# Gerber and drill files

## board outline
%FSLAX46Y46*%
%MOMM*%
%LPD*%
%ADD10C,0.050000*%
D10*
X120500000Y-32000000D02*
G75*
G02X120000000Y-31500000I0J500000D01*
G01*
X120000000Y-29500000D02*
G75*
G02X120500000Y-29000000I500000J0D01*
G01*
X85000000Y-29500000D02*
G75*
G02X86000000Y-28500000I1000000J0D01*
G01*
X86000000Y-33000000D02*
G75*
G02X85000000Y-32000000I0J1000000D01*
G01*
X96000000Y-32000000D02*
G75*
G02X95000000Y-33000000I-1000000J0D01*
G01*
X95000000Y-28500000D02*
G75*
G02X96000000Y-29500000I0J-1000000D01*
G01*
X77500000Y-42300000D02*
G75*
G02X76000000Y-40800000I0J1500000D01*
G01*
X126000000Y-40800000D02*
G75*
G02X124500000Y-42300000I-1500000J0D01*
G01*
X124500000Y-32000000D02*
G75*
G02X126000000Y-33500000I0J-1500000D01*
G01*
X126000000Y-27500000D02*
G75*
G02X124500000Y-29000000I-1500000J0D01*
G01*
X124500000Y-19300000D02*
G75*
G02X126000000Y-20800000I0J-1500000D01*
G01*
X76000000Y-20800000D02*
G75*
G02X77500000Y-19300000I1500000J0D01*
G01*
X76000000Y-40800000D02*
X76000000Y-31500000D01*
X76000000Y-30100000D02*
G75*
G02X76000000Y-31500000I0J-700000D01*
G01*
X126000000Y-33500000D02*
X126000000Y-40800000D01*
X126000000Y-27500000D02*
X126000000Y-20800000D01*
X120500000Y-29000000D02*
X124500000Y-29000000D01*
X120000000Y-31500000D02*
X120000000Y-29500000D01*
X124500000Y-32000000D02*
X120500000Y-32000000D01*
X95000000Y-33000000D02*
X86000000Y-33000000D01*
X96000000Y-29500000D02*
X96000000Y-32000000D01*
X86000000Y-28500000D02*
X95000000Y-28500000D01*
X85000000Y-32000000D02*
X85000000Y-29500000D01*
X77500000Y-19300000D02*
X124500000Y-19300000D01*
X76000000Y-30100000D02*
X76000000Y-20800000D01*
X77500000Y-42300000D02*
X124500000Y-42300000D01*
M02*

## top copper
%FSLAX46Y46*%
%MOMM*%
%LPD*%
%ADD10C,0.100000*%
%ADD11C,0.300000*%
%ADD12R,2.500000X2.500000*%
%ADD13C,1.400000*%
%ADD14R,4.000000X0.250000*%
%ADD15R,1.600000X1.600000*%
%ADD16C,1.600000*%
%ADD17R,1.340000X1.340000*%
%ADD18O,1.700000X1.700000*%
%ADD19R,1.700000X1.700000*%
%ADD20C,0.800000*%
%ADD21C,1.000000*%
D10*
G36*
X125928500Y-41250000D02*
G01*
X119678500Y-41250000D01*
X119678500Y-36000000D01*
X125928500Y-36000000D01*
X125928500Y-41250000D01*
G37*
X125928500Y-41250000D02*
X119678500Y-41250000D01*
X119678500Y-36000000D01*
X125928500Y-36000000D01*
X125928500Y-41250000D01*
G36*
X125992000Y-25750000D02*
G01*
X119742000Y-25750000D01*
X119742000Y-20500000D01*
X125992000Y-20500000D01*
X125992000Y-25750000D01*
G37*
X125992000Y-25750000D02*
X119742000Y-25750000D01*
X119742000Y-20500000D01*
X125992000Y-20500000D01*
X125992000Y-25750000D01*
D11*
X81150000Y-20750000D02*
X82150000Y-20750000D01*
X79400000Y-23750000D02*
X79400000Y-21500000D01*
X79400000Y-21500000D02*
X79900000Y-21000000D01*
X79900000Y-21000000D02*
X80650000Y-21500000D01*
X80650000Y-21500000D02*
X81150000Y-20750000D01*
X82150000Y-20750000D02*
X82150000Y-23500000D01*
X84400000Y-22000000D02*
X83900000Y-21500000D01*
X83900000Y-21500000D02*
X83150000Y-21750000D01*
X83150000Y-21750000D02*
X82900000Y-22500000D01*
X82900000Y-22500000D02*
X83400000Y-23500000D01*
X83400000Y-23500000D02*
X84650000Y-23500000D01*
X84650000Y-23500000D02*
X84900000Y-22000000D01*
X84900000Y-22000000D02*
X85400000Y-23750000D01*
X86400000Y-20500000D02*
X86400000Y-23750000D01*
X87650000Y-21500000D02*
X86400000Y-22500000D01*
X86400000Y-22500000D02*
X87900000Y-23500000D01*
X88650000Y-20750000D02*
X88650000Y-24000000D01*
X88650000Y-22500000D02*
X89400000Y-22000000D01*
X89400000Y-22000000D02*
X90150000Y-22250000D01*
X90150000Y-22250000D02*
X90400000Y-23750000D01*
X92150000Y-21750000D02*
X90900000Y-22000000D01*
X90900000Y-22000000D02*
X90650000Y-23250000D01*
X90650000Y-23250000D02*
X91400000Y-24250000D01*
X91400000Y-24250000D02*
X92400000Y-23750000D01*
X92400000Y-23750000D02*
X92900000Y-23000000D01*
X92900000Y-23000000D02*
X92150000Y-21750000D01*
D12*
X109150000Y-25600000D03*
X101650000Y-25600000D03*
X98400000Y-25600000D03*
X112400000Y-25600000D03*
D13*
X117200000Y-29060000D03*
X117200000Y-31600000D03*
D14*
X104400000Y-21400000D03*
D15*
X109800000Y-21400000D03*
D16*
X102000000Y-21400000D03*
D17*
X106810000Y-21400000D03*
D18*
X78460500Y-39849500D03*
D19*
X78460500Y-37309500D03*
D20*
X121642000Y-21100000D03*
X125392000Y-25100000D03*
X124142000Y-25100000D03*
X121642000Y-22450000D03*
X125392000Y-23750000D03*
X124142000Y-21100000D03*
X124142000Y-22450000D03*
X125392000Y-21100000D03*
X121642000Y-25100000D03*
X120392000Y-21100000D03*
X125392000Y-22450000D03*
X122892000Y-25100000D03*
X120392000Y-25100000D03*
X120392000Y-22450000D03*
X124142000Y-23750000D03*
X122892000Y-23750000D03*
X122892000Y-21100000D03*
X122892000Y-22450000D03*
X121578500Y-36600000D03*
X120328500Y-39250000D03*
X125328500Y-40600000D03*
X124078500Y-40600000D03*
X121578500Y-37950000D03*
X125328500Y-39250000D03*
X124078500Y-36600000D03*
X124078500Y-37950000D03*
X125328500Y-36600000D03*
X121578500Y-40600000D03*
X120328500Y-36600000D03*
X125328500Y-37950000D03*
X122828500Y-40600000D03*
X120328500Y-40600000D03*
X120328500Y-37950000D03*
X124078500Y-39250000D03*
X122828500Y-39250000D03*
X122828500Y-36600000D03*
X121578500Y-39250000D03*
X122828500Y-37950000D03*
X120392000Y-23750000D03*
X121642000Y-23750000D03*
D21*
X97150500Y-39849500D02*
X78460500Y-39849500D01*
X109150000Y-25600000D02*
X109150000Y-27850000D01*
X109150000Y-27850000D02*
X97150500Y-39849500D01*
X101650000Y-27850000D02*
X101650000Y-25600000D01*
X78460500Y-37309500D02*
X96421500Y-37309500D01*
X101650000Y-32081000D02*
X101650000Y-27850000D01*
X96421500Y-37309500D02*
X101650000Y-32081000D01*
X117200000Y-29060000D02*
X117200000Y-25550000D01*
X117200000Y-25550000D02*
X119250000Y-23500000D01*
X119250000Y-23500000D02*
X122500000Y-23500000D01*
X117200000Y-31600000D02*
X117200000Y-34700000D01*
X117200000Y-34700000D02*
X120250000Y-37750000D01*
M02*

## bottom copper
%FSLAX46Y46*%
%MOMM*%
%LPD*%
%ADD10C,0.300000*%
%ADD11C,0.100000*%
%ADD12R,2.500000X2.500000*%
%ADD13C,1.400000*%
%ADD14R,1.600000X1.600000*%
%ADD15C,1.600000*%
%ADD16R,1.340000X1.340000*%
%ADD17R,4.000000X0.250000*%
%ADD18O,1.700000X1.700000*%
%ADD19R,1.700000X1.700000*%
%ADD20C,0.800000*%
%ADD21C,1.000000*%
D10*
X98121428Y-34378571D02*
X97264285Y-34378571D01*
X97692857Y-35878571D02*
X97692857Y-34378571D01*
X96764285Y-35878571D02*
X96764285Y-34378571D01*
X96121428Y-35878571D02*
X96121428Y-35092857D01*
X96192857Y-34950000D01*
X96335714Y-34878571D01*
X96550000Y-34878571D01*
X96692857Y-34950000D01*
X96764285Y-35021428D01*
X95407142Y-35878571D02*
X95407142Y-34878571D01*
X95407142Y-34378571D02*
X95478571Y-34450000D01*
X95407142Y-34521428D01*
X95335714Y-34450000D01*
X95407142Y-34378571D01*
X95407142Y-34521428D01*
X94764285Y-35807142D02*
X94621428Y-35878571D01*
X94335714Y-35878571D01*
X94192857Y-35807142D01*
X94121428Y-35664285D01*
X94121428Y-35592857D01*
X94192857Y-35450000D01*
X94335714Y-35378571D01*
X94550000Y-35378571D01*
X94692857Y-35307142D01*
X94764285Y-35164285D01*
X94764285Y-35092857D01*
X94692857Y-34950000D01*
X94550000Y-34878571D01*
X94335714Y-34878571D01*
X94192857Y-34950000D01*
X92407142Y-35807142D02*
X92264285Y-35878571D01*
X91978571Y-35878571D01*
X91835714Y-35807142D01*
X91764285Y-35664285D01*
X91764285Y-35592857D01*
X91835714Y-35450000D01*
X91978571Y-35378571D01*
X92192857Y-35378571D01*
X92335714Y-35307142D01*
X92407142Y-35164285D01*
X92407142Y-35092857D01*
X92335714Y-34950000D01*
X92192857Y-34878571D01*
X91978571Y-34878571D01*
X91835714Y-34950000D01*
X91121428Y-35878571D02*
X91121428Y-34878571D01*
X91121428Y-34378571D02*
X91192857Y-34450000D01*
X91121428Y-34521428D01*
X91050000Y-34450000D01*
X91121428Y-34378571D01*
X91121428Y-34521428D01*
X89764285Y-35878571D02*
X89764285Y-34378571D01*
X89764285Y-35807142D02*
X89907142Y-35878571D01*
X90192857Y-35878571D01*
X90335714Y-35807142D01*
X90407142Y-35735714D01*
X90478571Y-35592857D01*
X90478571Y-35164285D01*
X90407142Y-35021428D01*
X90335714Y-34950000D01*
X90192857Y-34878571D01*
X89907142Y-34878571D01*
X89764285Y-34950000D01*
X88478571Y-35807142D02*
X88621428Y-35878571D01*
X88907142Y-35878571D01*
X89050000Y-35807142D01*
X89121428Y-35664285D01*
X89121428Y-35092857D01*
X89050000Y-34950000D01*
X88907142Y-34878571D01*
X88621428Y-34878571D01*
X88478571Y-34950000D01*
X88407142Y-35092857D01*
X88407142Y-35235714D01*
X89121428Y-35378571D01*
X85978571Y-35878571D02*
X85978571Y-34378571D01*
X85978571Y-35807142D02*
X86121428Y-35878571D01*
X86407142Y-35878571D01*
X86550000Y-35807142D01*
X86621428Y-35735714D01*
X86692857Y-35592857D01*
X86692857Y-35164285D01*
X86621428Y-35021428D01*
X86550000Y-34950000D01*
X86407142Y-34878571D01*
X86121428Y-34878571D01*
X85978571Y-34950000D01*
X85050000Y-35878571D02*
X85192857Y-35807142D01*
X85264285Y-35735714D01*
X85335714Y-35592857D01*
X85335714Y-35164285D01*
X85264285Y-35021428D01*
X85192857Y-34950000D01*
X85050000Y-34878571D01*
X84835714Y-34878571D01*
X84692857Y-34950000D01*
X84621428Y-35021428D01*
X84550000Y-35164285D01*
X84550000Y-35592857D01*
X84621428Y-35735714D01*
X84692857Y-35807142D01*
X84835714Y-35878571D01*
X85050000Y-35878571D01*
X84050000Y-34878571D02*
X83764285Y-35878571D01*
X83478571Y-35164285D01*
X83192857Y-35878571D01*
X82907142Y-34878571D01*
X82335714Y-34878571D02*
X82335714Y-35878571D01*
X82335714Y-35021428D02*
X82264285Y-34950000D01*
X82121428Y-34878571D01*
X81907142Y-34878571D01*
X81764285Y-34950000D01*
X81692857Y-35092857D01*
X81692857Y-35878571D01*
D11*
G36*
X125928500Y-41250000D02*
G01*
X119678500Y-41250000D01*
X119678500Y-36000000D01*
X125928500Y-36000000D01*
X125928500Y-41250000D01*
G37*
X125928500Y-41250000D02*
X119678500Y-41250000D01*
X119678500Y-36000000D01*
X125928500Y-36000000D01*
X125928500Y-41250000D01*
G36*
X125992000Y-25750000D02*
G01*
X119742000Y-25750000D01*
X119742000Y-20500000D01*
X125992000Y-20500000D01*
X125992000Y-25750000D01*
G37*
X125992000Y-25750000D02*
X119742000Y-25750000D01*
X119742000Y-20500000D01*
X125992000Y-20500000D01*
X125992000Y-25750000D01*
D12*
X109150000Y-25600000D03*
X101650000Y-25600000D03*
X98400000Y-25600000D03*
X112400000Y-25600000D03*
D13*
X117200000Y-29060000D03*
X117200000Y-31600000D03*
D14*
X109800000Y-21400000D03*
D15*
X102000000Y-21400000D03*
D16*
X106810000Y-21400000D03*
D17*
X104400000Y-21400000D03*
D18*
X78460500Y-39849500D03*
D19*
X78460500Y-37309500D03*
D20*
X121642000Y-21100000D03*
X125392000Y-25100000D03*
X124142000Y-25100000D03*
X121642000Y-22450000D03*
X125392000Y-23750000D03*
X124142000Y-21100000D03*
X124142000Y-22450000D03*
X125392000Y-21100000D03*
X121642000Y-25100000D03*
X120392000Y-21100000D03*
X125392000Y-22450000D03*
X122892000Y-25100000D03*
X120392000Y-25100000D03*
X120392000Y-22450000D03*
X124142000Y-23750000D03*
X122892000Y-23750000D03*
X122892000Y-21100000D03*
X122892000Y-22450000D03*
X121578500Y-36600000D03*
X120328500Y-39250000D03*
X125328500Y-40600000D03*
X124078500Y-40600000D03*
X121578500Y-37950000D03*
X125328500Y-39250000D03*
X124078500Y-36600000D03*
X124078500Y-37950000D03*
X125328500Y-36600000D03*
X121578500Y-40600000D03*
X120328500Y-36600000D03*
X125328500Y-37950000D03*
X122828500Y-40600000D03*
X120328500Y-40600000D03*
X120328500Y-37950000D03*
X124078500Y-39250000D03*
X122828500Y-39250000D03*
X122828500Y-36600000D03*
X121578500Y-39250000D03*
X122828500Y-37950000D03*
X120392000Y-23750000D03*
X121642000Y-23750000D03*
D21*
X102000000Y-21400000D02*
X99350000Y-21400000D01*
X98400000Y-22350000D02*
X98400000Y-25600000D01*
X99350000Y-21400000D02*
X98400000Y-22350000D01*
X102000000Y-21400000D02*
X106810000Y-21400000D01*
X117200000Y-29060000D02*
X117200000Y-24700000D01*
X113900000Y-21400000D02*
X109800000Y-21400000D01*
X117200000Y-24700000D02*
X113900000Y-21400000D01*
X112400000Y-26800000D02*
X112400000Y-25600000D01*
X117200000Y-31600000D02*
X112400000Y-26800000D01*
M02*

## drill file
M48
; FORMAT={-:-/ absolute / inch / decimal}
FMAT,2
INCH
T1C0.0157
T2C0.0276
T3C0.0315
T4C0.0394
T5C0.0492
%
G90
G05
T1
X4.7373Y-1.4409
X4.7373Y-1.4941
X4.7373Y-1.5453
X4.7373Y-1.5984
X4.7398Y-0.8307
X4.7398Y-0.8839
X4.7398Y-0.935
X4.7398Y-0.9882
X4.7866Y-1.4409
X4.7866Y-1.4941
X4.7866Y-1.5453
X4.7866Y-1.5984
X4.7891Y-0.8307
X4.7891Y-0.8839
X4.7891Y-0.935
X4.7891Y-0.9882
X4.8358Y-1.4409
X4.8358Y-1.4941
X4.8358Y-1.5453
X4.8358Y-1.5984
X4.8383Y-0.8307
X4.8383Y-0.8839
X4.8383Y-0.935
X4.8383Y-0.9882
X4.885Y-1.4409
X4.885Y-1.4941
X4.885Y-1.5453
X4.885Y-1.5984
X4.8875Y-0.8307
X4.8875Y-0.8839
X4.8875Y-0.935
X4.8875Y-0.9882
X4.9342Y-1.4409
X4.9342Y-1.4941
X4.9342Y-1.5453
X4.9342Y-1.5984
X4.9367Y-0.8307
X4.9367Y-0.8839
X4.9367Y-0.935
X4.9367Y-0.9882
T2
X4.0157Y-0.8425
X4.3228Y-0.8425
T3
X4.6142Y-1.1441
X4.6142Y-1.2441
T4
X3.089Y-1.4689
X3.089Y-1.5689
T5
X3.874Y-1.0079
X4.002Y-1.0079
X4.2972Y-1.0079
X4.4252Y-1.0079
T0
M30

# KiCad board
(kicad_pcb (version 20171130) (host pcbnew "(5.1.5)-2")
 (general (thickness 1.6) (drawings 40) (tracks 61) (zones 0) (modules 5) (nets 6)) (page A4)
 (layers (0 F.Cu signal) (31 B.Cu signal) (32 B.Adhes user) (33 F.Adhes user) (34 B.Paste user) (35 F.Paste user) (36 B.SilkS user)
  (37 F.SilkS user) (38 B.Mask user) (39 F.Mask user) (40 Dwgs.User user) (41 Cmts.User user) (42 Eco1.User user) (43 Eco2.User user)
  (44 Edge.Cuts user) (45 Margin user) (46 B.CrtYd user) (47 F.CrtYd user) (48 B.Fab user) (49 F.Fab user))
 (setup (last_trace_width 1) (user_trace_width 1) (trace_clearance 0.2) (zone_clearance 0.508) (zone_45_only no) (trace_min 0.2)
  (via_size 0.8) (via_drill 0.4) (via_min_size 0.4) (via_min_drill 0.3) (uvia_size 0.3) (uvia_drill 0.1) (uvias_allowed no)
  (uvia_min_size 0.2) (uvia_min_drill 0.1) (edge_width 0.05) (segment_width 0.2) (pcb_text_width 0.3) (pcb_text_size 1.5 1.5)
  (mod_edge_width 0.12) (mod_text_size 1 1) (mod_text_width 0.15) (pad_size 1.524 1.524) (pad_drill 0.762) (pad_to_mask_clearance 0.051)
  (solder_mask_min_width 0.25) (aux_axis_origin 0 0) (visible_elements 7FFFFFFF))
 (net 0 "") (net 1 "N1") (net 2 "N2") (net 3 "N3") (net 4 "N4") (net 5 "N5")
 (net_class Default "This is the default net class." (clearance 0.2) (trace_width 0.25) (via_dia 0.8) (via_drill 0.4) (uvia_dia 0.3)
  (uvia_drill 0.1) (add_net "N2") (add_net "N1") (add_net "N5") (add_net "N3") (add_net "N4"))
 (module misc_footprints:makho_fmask (layer F.Cu) (at 85.9 22.5)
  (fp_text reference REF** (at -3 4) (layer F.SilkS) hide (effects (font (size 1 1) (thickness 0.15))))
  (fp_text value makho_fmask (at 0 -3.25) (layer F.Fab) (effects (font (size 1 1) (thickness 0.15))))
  (fp_line (start -4.75 -1.75) (end -3.75 -1.75) (layer F.Cu) (width 0.3))
  (fp_line (start -6.5 1.25) (end -6.5 -1) (layer F.Cu) (width 0.3))
  (fp_line (start -6.5 -1) (end -6 -1.5) (layer F.Cu) (width 0.3))
  (fp_line (start -6 -1.5) (end -5.25 -1) (layer F.Cu) (width 0.3))
  (fp_line (start -5.25 -1) (end -4.75 -1.75) (layer F.Cu) (width 0.3))
  (fp_line (start -3.75 -1.75) (end -3.75 1) (layer F.Cu) (width 0.3))
  (fp_line (start -1.5 -0.5) (end -2 -1) (layer F.Cu) (width 0.3))
  (fp_line (start -2 -1) (end -2.75 -0.75) (layer F.Cu) (width 0.3))
  (fp_line (start -2.75 -0.75) (end -3 0) (layer F.Cu) (width 0.3)) (fp_line (start -3 0) (end -2.5 1) (layer F.Cu) (width 0.3))
  (fp_line (start -2.5 1) (end -1.25 1) (layer F.Cu) (width 0.3))
  (fp_line (start -1.25 1) (end -1 -0.5) (layer F.Cu) (width 0.3))
  (fp_line (start -1 -0.5) (end -0.5 1.25) (layer F.Cu) (width 0.3))
  (fp_line (start 0.5 -2) (end 0.5 1.25) (layer F.Cu) (width 0.3))
  (fp_line (start 1.75 -1) (end 0.5 0) (layer F.Cu) (width 0.3)) (fp_line (start 0.5 0) (end 2 1) (layer F.Cu) (width 0.3))
  (fp_line (start 2.75 -1.75) (end 2.75 1.5) (layer F.Cu) (width 0.3))
  (fp_line (start 2.75 0) (end 3.5 -0.5) (layer F.Cu) (width 0.3))
  (fp_line (start 3.5 -0.5) (end 4.25 -0.25) (layer F.Cu) (width 0.3))
  (fp_line (start 4.25 -0.25) (end 4.5 1.25) (layer F.Cu) (width 0.3))
  (fp_line (start 6.25 -0.75) (end 5 -0.5) (layer F.Cu) (width 0.3))
  (fp_line (start 5 -0.5) (end 4.75 0.75) (layer F.Cu) (width 0.3))
  (fp_line (start 4.75 0.75) (end 5.5 1.75) (layer F.Cu) (width 0.3))
  (fp_line (start 5.5 1.75) (end 6.5 1.25) (layer F.Cu) (width 0.3))
  (fp_line (start 6.5 1.25) (end 7 0.5) (layer F.Cu) (width 0.3))
  (fp_line (start 7 0.5) (end 6.25 -0.75) (layer F.Cu) (width 0.3)))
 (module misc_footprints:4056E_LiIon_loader (layer F.Cu) (at 105.4 36.6 90)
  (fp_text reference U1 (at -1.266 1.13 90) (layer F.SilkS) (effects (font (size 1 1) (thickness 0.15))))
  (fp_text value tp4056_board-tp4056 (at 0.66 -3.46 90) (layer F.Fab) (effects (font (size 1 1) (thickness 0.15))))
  (pad 4 thru_hole rect (at 11 3.75 90) (size 2.5 2.5) (drill 1.25) (layers *.Cu *.Mask F.SilkS) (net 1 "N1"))
  (pad 3 thru_hole rect (at 11 -3.75 90) (size 2.5 2.5) (drill 1.25) (layers *.Cu *.Mask F.SilkS) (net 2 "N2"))
  (pad 5 thru_hole rect (at 11 -7 90) (size 2.5 2.5) (drill 1.25) (layers *.Cu *.Mask F.SilkS) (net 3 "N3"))
  (pad 6 thru_hole rect (at 11 7 90) (size 2.5 2.5) (drill 1.25) (layers *.Cu *.Mask F.SilkS) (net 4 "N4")))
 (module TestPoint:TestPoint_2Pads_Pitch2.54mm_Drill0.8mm (layer F.Cu) (at 117.2 31.6 90)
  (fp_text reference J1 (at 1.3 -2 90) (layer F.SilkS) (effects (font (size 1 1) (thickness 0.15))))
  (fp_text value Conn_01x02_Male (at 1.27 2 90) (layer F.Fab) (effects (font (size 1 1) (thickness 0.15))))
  (pad 2 thru_hole circle (at 2.54 0 90) (size 1.4 1.4) (drill 0.8) (layers *.Cu *.Mask) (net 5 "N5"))
  (pad 1 thru_hole circle (at 0 0 90) (size 1.4 1.4) (drill 0.8) (layers *.Cu *.Mask) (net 4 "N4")))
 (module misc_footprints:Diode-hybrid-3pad (layer F.Cu) (at 105.9 21.4)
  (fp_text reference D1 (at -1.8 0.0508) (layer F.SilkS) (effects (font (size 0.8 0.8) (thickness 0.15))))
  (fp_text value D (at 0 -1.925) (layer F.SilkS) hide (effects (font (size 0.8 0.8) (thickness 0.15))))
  (pad 2 smd rect (at -1.5 0) (size 4 0.25) (layers F.Cu) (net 3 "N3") (solder_mask_margin -999))
  (pad 1 thru_hole rect (at 3.9 0) (size 1.6 1.6) (drill 0.7) (layers *.Cu *.Mask F.SilkS) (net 5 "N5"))
  (pad 2 thru_hole circle (at -3.9 0) (size 1.6 1.6) (drill 0.7) (layers *.Cu *.Mask F.SilkS) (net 3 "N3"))
  (pad 2 smd rect (at 0.91 0) (size 1.34 1.34) (layers F.Cu F.Paste F.Mask) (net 3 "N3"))
  (pad 2 smd rect (at 0.91 0) (size 1.34 1.34) (layers B.Cu B.Paste B.Mask) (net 3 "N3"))
  (pad 2 smd rect (at -1.5 0) (size 4 0.25) (layers B.Cu) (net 3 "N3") (solder_mask_margin -999)))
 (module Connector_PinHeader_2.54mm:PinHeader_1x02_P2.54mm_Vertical (layer F.Cu) (at 78.4605 37.3095)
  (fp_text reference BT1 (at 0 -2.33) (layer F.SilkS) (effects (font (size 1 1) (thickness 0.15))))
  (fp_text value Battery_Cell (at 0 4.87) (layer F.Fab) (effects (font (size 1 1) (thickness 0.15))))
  (pad 2 thru_hole oval (at 0 2.54) (size 1.7 1.7) (drill 1) (layers *.Cu *.Mask) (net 1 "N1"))
  (pad 1 thru_hole rect (at 0 0) (size 1.7 1.7) (drill 1) (layers *.Cu *.Mask) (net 2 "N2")))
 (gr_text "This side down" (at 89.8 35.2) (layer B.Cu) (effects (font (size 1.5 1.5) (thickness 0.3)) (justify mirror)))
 (gr_poly (pts (xy 125.9285 41.25) (xy 119.6785 41.25) (xy 119.6785 36) (xy 125.9285 36)) (layer B.Cu) (width 0.1))
 (gr_poly (pts (xy 125.9285 41.25) (xy 119.6785 41.25) (xy 119.6785 36) (xy 125.9285 36)) (layer F.Cu) (width 0.1))
 (gr_poly (pts (xy 125.992 25.75) (xy 119.742 25.75) (xy 119.742 20.5) (xy 125.992 20.5)) (layer B.Cu) (width 0.1))
 (gr_arc (start 120.5 31.5) (end 120 31.5) (angle -90) (layer Edge.Cuts) (width 0.05))
 (gr_arc (start 120.5 29.5) (end 120.5 29) (angle -90) (layer Edge.Cuts) (width 0.05))
 (gr_poly (pts (xy 125.992 25.75) (xy 119.742 25.75) (xy 119.742 20.5) (xy 125.992 20.5)) (layer F.Cu) (width 0.1))
 (gr_arc (start 86 29.5) (end 86 28.5) (angle -90) (layer Edge.Cuts) (width 0.05))
 (gr_arc (start 86 32) (end 85 32) (angle -90) (layer Edge.Cuts) (width 0.05))
 (gr_arc (start 95 32) (end 95 33) (angle -90) (layer Edge.Cuts) (width 0.05))
 (gr_arc (start 95 29.5) (end 96 29.5) (angle -90) (layer Edge.Cuts) (width 0.05))
 (gr_arc (start 77.5 40.8) (end 76 40.8) (angle -90) (layer Edge.Cuts) (width 0.05))
 (gr_arc (start 124.5 40.8) (end 124.5 42.3) (angle -90) (layer Edge.Cuts) (width 0.05))
 (gr_arc (start 124.5 33.5) (end 126 33.5) (angle -90) (layer Edge.Cuts) (width 0.05))
 (gr_arc (start 124.5 27.5) (end 124.5 29) (angle -90) (layer Edge.Cuts) (width 0.05))
 (gr_arc (start 124.5 20.8) (end 126 20.8) (angle -90) (layer Edge.Cuts) (width 0.05))
 (gr_arc (start 77.5 20.8) (end 77.5 19.3) (angle -90) (layer Edge.Cuts) (width 0.05))
 (gr_line (start 76 40.8) (end 76 31.5) (layer Edge.Cuts) (width 0.05))
 (gr_arc (start 76 30.8) (end 76 31.5) (angle -180) (layer Edge.Cuts) (width 0.05))
 (gr_line (start 126 33.5) (end 126 40.8) (layer Edge.Cuts) (width 0.05))
 (gr_line (start 126 27.5) (end 126 20.8) (layer Edge.Cuts) (width 0.05))
 (gr_line (start 120.5 29) (end 124.5 29) (layer Edge.Cuts) (width 0.05))
 (gr_line (start 120 31.5) (end 120 29.5) (layer Edge.Cuts) (width 0.05))
 (gr_line (start 124.5 32) (end 120.5 32) (layer Edge.Cuts) (width 0.05))
 (gr_line (start 95 33) (end 86 33) (layer Edge.Cuts) (width 0.05))
 (gr_line (start 96 29.5) (end 96 32) (layer Edge.Cuts) (width 0.05))
 (gr_line (start 86 28.5) (end 95 28.5) (layer Edge.Cuts) (width 0.05))
 (gr_line (start 85 32) (end 85 29.5) (layer Edge.Cuts) (width 0.05))
 (gr_line (start 77.5 19.3) (end 124.5 19.3) (layer Edge.Cuts) (width 0.05))
 (gr_line (start 76 30.1) (end 76 20.8) (layer Edge.Cuts) (width 0.05))
 (gr_line (start 77.5 42.3) (end 124.5 42.3) (layer Edge.Cuts) (width 0.05))
 (via (at 121.642 21.1) (size 0.8) (drill 0.4) (layers F.Cu B.Cu) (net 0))
 (via (at 125.392 25.1) (size 0.8) (drill 0.4) (layers F.Cu B.Cu) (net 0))
 (via (at 124.142 25.1) (size 0.8) (drill 0.4) (layers F.Cu B.Cu) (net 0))
 (via (at 121.642 22.45) (size 0.8) (drill 0.4) (layers F.Cu B.Cu) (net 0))
 (via (at 125.392 23.75) (size 0.8) (drill 0.4) (layers F.Cu B.Cu) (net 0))
 (via (at 124.142 21.1) (size 0.8) (drill 0.4) (layers F.Cu B.Cu) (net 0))
 (via (at 124.142 22.45) (size 0.8) (drill 0.4) (layers F.Cu B.Cu) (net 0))
 (via (at 125.392 21.1) (size 0.8) (drill 0.4) (layers F.Cu B.Cu) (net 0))
 (via (at 121.642 25.1) (size 0.8) (drill 0.4) (layers F.Cu B.Cu) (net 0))
 (via (at 120.392 21.1) (size 0.8) (drill 0.4) (layers F.Cu B.Cu) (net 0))
 (via (at 125.392 22.45) (size 0.8) (drill 0.4) (layers F.Cu B.Cu) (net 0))
 (via (at 122.892 25.1) (size 0.8) (drill 0.4) (layers F.Cu B.Cu) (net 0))
 (via (at 120.392 25.1) (size 0.8) (drill 0.4) (layers F.Cu B.Cu) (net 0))
 (via (at 120.392 22.45) (size 0.8) (drill 0.4) (layers F.Cu B.Cu) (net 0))
 (via (at 124.142 23.75) (size 0.8) (drill 0.4) (layers F.Cu B.Cu) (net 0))
 (via (at 122.892 23.75) (size 0.8) (drill 0.4) (layers F.Cu B.Cu) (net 5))
 (via (at 122.892 21.1) (size 0.8) (drill 0.4) (layers F.Cu B.Cu) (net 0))
 (via (at 122.892 22.45) (size 0.8) (drill 0.4) (layers F.Cu B.Cu) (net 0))
 (via (at 121.5785 36.6) (size 0.8) (drill 0.4) (layers F.Cu B.Cu) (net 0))
 (via (at 120.3285 39.25) (size 0.8) (drill 0.4) (layers F.Cu B.Cu) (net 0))
 (via (at 125.3285 40.6) (size 0.8) (drill 0.4) (layers F.Cu B.Cu) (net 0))
 (via (at 124.0785 40.6) (size 0.8) (drill 0.4) (layers F.Cu B.Cu) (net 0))
 (via (at 121.5785 37.95) (size 0.8) (drill 0.4) (layers F.Cu B.Cu) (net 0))
 (via (at 125.3285 39.25) (size 0.8) (drill 0.4) (layers F.Cu B.Cu) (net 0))
 (via (at 124.0785 36.6) (size 0.8) (drill 0.4) (layers F.Cu B.Cu) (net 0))
 (via (at 124.0785 37.95) (size 0.8) (drill 0.4) (layers F.Cu B.Cu) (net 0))
 (via (at 125.3285 36.6) (size 0.8) (drill 0.4) (layers F.Cu B.Cu) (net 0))
 (via (at 121.5785 40.6) (size 0.8) (drill 0.4) (layers F.Cu B.Cu) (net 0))
 (via (at 120.3285 36.6) (size 0.8) (drill 0.4) (layers F.Cu B.Cu) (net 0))
 (via (at 125.3285 37.95) (size 0.8) (drill 0.4) (layers F.Cu B.Cu) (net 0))
 (via (at 122.8285 40.6) (size 0.8) (drill 0.4) (layers F.Cu B.Cu) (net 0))
 (via (at 120.3285 40.6) (size 0.8) (drill 0.4) (layers F.Cu B.Cu) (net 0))
 (via (at 120.3285 37.95) (size 0.8) (drill 0.4) (layers F.Cu B.Cu) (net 4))
 (via (at 124.0785 39.25) (size 0.8) (drill 0.4) (layers F.Cu B.Cu) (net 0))
 (via (at 122.8285 39.25) (size 0.8) (drill 0.4) (layers F.Cu B.Cu) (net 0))
 (via (at 122.8285 36.6) (size 0.8) (drill 0.4) (layers F.Cu B.Cu) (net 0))
 (via (at 121.5785 39.25) (size 0.8) (drill 0.4) (layers F.Cu B.Cu) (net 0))
 (via (at 122.8285 37.95) (size 0.8) (drill 0.4) (layers F.Cu B.Cu) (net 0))
 (segment (start 97.1505 39.8495) (end 78.4605 39.8495) (width 1) (layer F.Cu) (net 1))
 (segment (start 109.15 25.6) (end 109.15 27.85) (width 1) (layer F.Cu) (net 1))
 (segment (start 109.15 27.85) (end 97.1505 39.8495) (width 1) (layer F.Cu) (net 1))
 (segment (start 101.65 27.85) (end 101.65 25.6) (width 1) (layer F.Cu) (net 2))
 (segment (start 78.4605 37.3095) (end 96.4215 37.3095) (width 1) (layer F.Cu) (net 2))
 (segment (start 101.65 32.081) (end 101.65 27.85) (width 1) (layer F.Cu) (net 2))
 (segment (start 96.4215 37.3095) (end 101.65 32.081) (width 1) (layer F.Cu) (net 2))
 (segment (start 102 21.4) (end 99.35 21.4) (width 1) (layer B.Cu) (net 3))
 (segment (start 98.4 22.35) (end 98.4 25.6) (width 1) (layer B.Cu) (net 3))
 (segment (start 99.35 21.4) (end 98.4 22.35) (width 1) (layer B.Cu) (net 3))
 (segment (start 102 21.4) (end 106.81 21.4) (width 1) (layer B.Cu) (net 3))
 (via (at 120.392 23.75) (size 0.8) (drill 0.4) (layers F.Cu B.Cu) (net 5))
 (via (at 121.642 23.75) (size 0.8) (drill 0.4) (layers F.Cu B.Cu) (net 5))
 (segment (start 117.2 29.06) (end 117.2 25.55) (width 1) (layer F.Cu) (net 5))
 (segment (start 117.2 25.55) (end 119.25 23.5) (width 1) (layer F.Cu) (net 5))
 (segment (start 117.2 29.06) (end 117.2 24.7) (width 1) (layer B.Cu) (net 5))
 (segment (start 113.9 21.4) (end 109.8 21.4) (width 1) (layer B.Cu) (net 5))
 (segment (start 117.2 24.7) (end 113.9 21.4) (width 1) (layer B.Cu) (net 5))
 (segment (start 119.25 23.5) (end 122.5 23.5) (width 1) (layer F.Cu) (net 5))
 (segment (start 117.2 31.6) (end 117.2 34.7) (width 1) (layer F.Cu) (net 4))
 (segment (start 117.2 34.7) (end 120.25 37.75) (width 1) (layer F.Cu) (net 4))
 (segment (start 112.4 26.8) (end 112.4 25.6) (width 1) (layer B.Cu) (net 4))
 (segment (start 117.2 31.6) (end 112.4 26.8) (width 1) (layer B.Cu) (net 4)))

